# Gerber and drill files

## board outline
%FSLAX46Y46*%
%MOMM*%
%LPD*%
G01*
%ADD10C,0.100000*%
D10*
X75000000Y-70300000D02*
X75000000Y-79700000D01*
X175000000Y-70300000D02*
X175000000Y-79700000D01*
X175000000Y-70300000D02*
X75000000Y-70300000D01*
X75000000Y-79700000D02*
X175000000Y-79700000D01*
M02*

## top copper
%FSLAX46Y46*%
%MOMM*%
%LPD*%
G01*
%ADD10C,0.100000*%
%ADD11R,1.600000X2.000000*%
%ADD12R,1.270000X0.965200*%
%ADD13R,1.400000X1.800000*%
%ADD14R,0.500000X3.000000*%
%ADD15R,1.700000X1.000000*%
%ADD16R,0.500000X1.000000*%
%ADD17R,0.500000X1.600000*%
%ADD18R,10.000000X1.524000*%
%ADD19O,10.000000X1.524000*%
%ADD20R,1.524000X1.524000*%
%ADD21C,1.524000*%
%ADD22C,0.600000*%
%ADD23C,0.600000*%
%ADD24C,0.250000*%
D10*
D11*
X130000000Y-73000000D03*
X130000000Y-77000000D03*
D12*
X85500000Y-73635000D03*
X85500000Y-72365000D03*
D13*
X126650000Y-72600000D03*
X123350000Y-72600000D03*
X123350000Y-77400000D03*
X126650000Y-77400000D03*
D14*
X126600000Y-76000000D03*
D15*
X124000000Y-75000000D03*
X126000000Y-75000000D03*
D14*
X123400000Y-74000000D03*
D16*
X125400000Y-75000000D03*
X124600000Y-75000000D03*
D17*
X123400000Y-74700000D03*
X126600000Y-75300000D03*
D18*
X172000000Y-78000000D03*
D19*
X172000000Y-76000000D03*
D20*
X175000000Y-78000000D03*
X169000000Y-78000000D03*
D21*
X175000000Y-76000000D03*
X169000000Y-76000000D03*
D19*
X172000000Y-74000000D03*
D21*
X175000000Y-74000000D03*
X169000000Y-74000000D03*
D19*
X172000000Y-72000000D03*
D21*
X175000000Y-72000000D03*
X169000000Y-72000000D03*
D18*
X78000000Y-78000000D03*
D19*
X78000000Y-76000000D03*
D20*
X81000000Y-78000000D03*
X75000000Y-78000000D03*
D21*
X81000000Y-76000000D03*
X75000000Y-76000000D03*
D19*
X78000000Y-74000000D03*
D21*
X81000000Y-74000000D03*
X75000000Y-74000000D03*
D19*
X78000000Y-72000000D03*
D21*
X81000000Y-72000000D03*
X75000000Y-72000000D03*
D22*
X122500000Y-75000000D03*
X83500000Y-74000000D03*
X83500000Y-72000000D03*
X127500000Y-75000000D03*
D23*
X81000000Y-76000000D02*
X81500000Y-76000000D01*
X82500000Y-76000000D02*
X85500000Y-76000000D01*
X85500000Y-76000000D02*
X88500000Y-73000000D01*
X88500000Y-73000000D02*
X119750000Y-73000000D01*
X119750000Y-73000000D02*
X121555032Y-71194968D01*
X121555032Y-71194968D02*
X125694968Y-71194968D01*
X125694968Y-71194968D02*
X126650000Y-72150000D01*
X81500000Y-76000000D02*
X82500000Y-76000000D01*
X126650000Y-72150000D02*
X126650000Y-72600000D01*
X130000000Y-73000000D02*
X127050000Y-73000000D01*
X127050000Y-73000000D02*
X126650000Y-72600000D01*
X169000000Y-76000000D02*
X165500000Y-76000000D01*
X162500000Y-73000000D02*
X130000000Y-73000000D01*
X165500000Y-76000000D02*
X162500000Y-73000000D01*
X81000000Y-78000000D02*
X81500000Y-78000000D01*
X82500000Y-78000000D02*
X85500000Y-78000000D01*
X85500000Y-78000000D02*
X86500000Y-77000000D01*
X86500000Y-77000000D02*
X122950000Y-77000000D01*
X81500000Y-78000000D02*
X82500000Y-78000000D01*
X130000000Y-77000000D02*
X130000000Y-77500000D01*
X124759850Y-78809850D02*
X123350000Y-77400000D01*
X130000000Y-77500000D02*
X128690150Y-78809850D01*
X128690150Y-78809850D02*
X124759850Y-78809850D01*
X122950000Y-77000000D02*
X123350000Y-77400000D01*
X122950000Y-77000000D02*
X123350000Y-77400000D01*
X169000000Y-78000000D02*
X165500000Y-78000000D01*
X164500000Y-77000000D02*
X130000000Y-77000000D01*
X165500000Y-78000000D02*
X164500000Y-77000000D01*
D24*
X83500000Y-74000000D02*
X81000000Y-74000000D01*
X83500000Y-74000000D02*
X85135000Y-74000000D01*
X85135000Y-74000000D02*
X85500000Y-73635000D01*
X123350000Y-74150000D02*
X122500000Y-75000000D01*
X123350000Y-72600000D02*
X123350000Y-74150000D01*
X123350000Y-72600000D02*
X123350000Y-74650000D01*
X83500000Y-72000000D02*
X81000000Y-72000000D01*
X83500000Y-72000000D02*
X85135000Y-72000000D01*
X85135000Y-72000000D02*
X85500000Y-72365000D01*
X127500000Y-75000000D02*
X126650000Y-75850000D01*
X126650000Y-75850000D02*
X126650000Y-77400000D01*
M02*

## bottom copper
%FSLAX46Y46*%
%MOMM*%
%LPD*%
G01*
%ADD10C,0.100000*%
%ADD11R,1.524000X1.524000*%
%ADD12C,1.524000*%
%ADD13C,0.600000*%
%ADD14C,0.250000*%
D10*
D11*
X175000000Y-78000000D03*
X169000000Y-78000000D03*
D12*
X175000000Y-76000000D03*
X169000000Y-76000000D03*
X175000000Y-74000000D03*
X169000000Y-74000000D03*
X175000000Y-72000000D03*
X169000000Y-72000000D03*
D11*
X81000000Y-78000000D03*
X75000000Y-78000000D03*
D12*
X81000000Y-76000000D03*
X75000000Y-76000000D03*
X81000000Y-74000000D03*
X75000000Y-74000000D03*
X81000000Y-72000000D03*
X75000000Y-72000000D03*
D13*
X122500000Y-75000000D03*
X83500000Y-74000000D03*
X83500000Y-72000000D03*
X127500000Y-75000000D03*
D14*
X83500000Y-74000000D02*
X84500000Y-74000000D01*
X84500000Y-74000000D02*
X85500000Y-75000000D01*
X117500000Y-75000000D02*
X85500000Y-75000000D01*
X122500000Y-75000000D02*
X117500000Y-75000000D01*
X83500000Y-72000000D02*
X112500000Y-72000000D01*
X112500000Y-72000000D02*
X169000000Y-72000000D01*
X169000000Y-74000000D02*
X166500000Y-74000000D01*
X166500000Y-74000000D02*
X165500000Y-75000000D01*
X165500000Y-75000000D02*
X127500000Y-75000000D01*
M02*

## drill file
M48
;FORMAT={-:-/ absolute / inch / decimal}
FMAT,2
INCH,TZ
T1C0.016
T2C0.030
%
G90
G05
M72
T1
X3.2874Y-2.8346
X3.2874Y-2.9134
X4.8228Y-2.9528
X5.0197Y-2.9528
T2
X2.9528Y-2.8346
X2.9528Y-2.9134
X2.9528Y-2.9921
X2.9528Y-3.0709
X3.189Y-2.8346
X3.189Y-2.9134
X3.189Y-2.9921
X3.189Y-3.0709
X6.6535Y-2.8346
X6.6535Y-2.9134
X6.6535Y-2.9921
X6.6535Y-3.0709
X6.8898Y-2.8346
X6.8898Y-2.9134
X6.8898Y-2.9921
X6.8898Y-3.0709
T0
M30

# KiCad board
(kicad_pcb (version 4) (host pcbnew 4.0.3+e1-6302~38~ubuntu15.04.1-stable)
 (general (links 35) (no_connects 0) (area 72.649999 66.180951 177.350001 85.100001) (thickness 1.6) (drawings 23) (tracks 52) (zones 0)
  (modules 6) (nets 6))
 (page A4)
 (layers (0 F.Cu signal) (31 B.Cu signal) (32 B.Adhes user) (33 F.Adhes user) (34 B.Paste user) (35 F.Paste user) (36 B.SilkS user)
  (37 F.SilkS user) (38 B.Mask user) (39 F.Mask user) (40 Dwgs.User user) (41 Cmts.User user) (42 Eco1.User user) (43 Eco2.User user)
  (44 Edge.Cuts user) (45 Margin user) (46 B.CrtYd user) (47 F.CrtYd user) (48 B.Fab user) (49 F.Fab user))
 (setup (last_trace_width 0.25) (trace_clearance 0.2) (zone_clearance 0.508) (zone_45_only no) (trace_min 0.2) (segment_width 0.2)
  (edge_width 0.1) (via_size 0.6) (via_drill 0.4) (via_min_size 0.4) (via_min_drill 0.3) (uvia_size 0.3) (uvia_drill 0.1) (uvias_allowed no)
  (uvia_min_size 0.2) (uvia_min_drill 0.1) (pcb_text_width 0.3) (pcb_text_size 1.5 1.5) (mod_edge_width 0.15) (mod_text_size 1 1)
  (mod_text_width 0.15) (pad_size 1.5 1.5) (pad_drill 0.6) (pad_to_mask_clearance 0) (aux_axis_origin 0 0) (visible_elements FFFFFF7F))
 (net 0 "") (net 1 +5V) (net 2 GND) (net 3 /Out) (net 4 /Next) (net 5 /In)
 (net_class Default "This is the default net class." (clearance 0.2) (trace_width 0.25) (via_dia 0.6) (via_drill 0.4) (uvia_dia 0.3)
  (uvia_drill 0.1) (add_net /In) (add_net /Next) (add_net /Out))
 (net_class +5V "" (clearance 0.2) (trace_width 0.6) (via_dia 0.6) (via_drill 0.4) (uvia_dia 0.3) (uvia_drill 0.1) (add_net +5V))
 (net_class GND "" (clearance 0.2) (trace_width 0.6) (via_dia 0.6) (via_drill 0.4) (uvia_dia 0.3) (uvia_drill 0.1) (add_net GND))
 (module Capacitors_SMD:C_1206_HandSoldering (layer F.Cu) (at 130 75 270)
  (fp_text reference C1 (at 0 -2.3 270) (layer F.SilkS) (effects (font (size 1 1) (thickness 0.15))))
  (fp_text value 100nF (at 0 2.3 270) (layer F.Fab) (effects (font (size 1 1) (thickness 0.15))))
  (pad 1 smd rect (at -2 0 270) (size 2 1.6) (layers F.Cu F.Paste F.Mask) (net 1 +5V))
  (pad 2 smd rect (at 2 0 270) (size 2 1.6) (layers F.Cu F.Paste F.Mask) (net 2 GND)))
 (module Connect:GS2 (layer F.Cu) (at 85.5 73 180)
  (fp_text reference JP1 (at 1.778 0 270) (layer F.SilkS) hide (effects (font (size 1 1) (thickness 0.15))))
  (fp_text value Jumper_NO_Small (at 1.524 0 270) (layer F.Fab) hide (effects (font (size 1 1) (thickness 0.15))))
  (pad 1 smd rect (at 0 -0.635 180) (size 1.27 0.9652) (layers F.Cu F.Paste F.Mask) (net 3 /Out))
  (pad 2 smd rect (at 0 0.635 180) (size 1.27 0.9652) (layers F.Cu F.Paste F.Mask) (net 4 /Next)))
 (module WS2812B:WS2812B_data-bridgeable (layer F.Cu) (at 125 75)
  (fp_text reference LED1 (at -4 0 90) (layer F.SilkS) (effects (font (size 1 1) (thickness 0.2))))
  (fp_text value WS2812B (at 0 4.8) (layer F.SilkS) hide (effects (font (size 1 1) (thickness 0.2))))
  (pad 1 smd rect (at 1.65 -2.4) (size 1.4 1.8) (layers F.Cu F.Paste F.Mask) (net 1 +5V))
  (pad 2 smd rect (at -1.65 -2.4) (size 1.4 1.8) (layers F.Cu F.Paste F.Mask) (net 3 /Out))
  (pad 3 smd rect (at -1.65 2.4) (size 1.4 1.8) (layers F.Cu F.Paste F.Mask) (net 2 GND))
  (pad 4 smd rect (at 1.65 2.4) (size 1.4 1.8) (layers F.Cu F.Paste F.Mask) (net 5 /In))
  (pad 4 smd rect (at 1.6 1) (size 0.5 3) (layers F.Cu) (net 5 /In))
  (pad 2 smd rect (at -1 0) (size 1.7 1) (layers F.Cu) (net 3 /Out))
  (pad 4 smd rect (at 1 0) (size 1.7 1) (layers F.Cu) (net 5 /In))
  (pad 2 smd rect (at -1.6 -1) (size 0.5 3) (layers F.Cu) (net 3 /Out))
  (pad 4 smd rect (at 0.4 0) (size 0.5 1) (layers F.Cu F.Mask) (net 5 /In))
  (pad 2 smd rect (at -0.4 0) (size 0.5 1) (layers F.Cu F.Mask) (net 3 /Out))
  (pad 2 smd rect (at -1.6 -0.3) (size 0.5 1.6) (layers F.Cu) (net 3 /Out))
  (pad 4 smd rect (at 1.6 0.3) (size 0.5 1.6) (layers F.Cu) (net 5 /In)))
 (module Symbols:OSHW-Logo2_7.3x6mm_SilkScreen (layer F.Cu) (at 111 75.5)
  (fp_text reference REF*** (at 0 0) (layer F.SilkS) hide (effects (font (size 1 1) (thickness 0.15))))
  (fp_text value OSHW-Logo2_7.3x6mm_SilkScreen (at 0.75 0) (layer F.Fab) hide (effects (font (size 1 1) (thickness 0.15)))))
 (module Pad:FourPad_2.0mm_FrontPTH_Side (layer F.Cu) (at 172 75)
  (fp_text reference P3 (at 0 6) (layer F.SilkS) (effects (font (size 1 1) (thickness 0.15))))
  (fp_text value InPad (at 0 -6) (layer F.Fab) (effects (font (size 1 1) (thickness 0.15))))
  (pad 1 smd rect (at 0 3) (size 10 1.524) (layers F.Cu F.Paste F.Mask) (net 2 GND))
  (pad 2 smd oval (at 0 1) (size 10 1.524) (layers F.Cu F.Paste F.Mask) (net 1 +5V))
  (pad 1 thru_hole rect (at 3 3) (size 1.524 1.524) (drill 0.762) (layers *.Cu F.Mask) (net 2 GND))
  (pad 1 thru_hole rect (at -3 3) (size 1.524 1.524) (drill 0.762) (layers *.Cu F.Mask) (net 2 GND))
  (pad 2 thru_hole circle (at 3 1) (size 1.524 1.524) (drill 0.762) (layers *.Cu F.Mask) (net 1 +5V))
  (pad 2 thru_hole circle (at -3 1) (size 1.524 1.524) (drill 0.762) (layers *.Cu F.Mask) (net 1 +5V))
  (pad 3 smd oval (at 0 -1) (size 10 1.524) (layers F.Cu F.Paste F.Mask) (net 5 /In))
  (pad 3 thru_hole circle (at 3 -1) (size 1.524 1.524) (drill 0.762) (layers *.Cu F.Mask) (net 5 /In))
  (pad 3 thru_hole circle (at -3 -1) (size 1.524 1.524) (drill 0.762) (layers *.Cu F.Mask) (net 5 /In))
  (pad 4 smd oval (at 0 -3) (size 10 1.524) (layers F.Cu F.Paste F.Mask) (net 4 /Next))
  (pad 4 thru_hole circle (at 3 -3) (size 1.524 1.524) (drill 0.762) (layers *.Cu F.Mask) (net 4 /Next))
  (pad 4 thru_hole circle (at -3 -3) (size 1.524 1.524) (drill 0.762) (layers *.Cu F.Mask) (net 4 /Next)))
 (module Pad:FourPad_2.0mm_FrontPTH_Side (layer F.Cu) (at 78 75)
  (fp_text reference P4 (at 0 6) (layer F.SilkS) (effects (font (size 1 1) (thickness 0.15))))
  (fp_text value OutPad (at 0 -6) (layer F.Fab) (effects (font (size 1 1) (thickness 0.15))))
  (pad 1 smd rect (at 0 3) (size 10 1.524) (layers F.Cu F.Paste F.Mask) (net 2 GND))
  (pad 2 smd oval (at 0 1) (size 10 1.524) (layers F.Cu F.Paste F.Mask) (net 1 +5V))
  (pad 1 thru_hole rect (at 3 3) (size 1.524 1.524) (drill 0.762) (layers *.Cu F.Mask) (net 2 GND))
  (pad 1 thru_hole rect (at -3 3) (size 1.524 1.524) (drill 0.762) (layers *.Cu F.Mask) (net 2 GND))
  (pad 2 thru_hole circle (at 3 1) (size 1.524 1.524) (drill 0.762) (layers *.Cu F.Mask) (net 1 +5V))
  (pad 2 thru_hole circle (at -3 1) (size 1.524 1.524) (drill 0.762) (layers *.Cu F.Mask) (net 1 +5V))
  (pad 3 smd oval (at 0 -1) (size 10 1.524) (layers F.Cu F.Paste F.Mask) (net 3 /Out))
  (pad 3 thru_hole circle (at 3 -1) (size 1.524 1.524) (drill 0.762) (layers *.Cu F.Mask) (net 3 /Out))
  (pad 3 thru_hole circle (at -3 -1) (size 1.524 1.524) (drill 0.762) (layers *.Cu F.Mask) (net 3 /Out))
  (pad 4 smd oval (at 0 -3) (size 10 1.524) (layers F.Cu F.Paste F.Mask) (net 4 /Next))
  (pad 4 thru_hole circle (at 3 -3) (size 1.524 1.524) (drill 0.762) (layers *.Cu F.Mask) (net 4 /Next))
  (pad 4 thru_hole circle (at -3 -3) (size 1.524 1.524) (drill 0.762) (layers *.Cu F.Mask) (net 4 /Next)))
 (gr_line (start 75 70.3) (end 75 79.7) (angle 90) (layer Edge.Cuts) (width 0.1))
 (gr_line (start 175 70.3) (end 175 79.7) (angle 90) (layer Edge.Cuts) (width 0.1))
 (gr_line (start 175 70.3) (end 75 70.3) (angle 90) (layer Edge.Cuts) (width 0.1))
 (gr_line (start 75 79.7) (end 175 79.7) (angle 90) (layer Edge.Cuts) (width 0.1))
 (segment (start 81 76) (end 81.5 76) (width 0.6) (layer F.Cu) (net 1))
 (segment (start 82.5 76) (end 85.5 76) (width 0.6) (layer F.Cu) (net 1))
 (segment (start 85.5 76) (end 88.5 73) (width 0.6) (layer F.Cu) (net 1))
 (segment (start 88.5 73) (end 119.75 73) (width 0.6) (layer F.Cu) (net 1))
 (segment (start 119.75 73) (end 121.555032 71.194968) (width 0.6) (layer F.Cu) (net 1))
 (segment (start 121.555032 71.194968) (end 125.694968 71.194968) (width 0.6) (layer F.Cu) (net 1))
 (segment (start 125.694968 71.194968) (end 126.65 72.15) (width 0.6) (layer F.Cu) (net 1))
 (segment (start 81.5 76) (end 82.5 76) (width 0.6) (layer F.Cu) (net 1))
 (segment (start 126.65 72.15) (end 126.65 72.6) (width 0.6) (layer F.Cu) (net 1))
 (segment (start 130 73) (end 127.05 73) (width 0.6) (layer F.Cu) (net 1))
 (segment (start 127.05 73) (end 126.65 72.6) (width 0.6) (layer F.Cu) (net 1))
 (segment (start 169 76) (end 165.5 76) (width 0.6) (layer F.Cu) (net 1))
 (segment (start 162.5 73) (end 130 73) (width 0.6) (layer F.Cu) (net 1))
 (segment (start 165.5 76) (end 162.5 73) (width 0.6) (layer F.Cu) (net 1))
 (segment (start 81 78) (end 81.5 78) (width 0.6) (layer F.Cu) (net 2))
 (segment (start 82.5 78) (end 85.5 78) (width 0.6) (layer F.Cu) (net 2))
 (segment (start 85.5 78) (end 86.5 77) (width 0.6) (layer F.Cu) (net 2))
 (segment (start 86.5 77) (end 122.95 77) (width 0.6) (layer F.Cu) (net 2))
 (segment (start 81.5 78) (end 82.5 78) (width 0.6) (layer F.Cu) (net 2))
 (segment (start 130 77) (end 130 77.5) (width 0.6) (layer F.Cu) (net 2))
 (segment (start 124.75985 78.80985) (end 123.35 77.4) (width 0.6) (layer F.Cu) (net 2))
 (segment (start 130 77.5) (end 128.69015 78.80985) (width 0.6) (layer F.Cu) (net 2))
 (segment (start 128.69015 78.80985) (end 124.75985 78.80985) (width 0.6) (layer F.Cu) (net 2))
 (segment (start 122.95 77) (end 123.35 77.4) (width 0.6) (layer F.Cu) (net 2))
 (segment (start 122.95 77) (end 123.35 77.4) (width 0.6) (layer F.Cu) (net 2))
 (segment (start 169 78) (end 165.5 78) (width 0.6) (layer F.Cu) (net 2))
 (segment (start 164.5 77) (end 130 77) (width 0.6) (layer F.Cu) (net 2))
 (segment (start 165.5 78) (end 164.5 77) (width 0.6) (layer F.Cu) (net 2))
 (segment (start 83.5 74) (end 81 74) (width 0.25) (layer F.Cu) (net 3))
 (segment (start 83.5 74) (end 84.5 74) (width 0.25) (layer B.Cu) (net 3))
 (segment (start 84.5 74) (end 85.5 75) (width 0.25) (layer B.Cu) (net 3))
 (segment (start 83.5 74) (end 85.135 74) (width 0.25) (layer F.Cu) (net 3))
 (segment (start 85.135 74) (end 85.5 73.635) (width 0.25) (layer F.Cu) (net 3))
 (segment (start 117.5 75) (end 85.5 75) (width 0.25) (layer B.Cu) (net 3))
 (via (at 122.5 75) (size 0.6) (drill 0.4) (layers F.Cu B.Cu) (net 3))
 (segment (start 123.35 74.15) (end 122.5 75) (width 0.25) (layer F.Cu) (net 3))
 (segment (start 122.5 75) (end 117.5 75) (width 0.25) (layer B.Cu) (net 3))
 (via (at 83.5 74) (size 0.6) (drill 0.4) (layers F.Cu B.Cu) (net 3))
 (segment (start 123.35 72.6) (end 123.35 74.15) (width 0.25) (layer F.Cu) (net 3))
 (segment (start 123.35 72.6) (end 123.35 74.65) (width 0.25) (layer F.Cu) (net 3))
 (segment (start 83.5 72) (end 81 72) (width 0.25) (layer F.Cu) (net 4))
 (segment (start 83.5 72) (end 85.135 72) (width 0.25) (layer F.Cu) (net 4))
 (segment (start 85.135 72) (end 85.5 72.365) (width 0.25) (layer F.Cu) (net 4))
 (segment (start 83.5 72) (end 112.5 72) (width 0.25) (layer B.Cu) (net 4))
 (via (at 83.5 72) (size 0.6) (drill 0.4) (layers F.Cu B.Cu) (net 4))
 (segment (start 112.5 72) (end 169 72) (width 0.25) (layer B.Cu) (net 4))
 (segment (start 169 74) (end 166.5 74) (width 0.25) (layer B.Cu) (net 5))
 (segment (start 166.5 74) (end 165.5 75) (width 0.25) (layer B.Cu) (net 5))
 (segment (start 127.5 75) (end 126.65 75.85) (width 0.25) (layer F.Cu) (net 5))
 (via (at 127.5 75) (size 0.6) (drill 0.4) (layers F.Cu B.Cu) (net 5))
 (segment (start 165.5 75) (end 127.5 75) (width 0.25) (layer B.Cu) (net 5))
 (segment (start 126.65 75.85) (end 126.65 77.4) (width 0.25) (layer F.Cu) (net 5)))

